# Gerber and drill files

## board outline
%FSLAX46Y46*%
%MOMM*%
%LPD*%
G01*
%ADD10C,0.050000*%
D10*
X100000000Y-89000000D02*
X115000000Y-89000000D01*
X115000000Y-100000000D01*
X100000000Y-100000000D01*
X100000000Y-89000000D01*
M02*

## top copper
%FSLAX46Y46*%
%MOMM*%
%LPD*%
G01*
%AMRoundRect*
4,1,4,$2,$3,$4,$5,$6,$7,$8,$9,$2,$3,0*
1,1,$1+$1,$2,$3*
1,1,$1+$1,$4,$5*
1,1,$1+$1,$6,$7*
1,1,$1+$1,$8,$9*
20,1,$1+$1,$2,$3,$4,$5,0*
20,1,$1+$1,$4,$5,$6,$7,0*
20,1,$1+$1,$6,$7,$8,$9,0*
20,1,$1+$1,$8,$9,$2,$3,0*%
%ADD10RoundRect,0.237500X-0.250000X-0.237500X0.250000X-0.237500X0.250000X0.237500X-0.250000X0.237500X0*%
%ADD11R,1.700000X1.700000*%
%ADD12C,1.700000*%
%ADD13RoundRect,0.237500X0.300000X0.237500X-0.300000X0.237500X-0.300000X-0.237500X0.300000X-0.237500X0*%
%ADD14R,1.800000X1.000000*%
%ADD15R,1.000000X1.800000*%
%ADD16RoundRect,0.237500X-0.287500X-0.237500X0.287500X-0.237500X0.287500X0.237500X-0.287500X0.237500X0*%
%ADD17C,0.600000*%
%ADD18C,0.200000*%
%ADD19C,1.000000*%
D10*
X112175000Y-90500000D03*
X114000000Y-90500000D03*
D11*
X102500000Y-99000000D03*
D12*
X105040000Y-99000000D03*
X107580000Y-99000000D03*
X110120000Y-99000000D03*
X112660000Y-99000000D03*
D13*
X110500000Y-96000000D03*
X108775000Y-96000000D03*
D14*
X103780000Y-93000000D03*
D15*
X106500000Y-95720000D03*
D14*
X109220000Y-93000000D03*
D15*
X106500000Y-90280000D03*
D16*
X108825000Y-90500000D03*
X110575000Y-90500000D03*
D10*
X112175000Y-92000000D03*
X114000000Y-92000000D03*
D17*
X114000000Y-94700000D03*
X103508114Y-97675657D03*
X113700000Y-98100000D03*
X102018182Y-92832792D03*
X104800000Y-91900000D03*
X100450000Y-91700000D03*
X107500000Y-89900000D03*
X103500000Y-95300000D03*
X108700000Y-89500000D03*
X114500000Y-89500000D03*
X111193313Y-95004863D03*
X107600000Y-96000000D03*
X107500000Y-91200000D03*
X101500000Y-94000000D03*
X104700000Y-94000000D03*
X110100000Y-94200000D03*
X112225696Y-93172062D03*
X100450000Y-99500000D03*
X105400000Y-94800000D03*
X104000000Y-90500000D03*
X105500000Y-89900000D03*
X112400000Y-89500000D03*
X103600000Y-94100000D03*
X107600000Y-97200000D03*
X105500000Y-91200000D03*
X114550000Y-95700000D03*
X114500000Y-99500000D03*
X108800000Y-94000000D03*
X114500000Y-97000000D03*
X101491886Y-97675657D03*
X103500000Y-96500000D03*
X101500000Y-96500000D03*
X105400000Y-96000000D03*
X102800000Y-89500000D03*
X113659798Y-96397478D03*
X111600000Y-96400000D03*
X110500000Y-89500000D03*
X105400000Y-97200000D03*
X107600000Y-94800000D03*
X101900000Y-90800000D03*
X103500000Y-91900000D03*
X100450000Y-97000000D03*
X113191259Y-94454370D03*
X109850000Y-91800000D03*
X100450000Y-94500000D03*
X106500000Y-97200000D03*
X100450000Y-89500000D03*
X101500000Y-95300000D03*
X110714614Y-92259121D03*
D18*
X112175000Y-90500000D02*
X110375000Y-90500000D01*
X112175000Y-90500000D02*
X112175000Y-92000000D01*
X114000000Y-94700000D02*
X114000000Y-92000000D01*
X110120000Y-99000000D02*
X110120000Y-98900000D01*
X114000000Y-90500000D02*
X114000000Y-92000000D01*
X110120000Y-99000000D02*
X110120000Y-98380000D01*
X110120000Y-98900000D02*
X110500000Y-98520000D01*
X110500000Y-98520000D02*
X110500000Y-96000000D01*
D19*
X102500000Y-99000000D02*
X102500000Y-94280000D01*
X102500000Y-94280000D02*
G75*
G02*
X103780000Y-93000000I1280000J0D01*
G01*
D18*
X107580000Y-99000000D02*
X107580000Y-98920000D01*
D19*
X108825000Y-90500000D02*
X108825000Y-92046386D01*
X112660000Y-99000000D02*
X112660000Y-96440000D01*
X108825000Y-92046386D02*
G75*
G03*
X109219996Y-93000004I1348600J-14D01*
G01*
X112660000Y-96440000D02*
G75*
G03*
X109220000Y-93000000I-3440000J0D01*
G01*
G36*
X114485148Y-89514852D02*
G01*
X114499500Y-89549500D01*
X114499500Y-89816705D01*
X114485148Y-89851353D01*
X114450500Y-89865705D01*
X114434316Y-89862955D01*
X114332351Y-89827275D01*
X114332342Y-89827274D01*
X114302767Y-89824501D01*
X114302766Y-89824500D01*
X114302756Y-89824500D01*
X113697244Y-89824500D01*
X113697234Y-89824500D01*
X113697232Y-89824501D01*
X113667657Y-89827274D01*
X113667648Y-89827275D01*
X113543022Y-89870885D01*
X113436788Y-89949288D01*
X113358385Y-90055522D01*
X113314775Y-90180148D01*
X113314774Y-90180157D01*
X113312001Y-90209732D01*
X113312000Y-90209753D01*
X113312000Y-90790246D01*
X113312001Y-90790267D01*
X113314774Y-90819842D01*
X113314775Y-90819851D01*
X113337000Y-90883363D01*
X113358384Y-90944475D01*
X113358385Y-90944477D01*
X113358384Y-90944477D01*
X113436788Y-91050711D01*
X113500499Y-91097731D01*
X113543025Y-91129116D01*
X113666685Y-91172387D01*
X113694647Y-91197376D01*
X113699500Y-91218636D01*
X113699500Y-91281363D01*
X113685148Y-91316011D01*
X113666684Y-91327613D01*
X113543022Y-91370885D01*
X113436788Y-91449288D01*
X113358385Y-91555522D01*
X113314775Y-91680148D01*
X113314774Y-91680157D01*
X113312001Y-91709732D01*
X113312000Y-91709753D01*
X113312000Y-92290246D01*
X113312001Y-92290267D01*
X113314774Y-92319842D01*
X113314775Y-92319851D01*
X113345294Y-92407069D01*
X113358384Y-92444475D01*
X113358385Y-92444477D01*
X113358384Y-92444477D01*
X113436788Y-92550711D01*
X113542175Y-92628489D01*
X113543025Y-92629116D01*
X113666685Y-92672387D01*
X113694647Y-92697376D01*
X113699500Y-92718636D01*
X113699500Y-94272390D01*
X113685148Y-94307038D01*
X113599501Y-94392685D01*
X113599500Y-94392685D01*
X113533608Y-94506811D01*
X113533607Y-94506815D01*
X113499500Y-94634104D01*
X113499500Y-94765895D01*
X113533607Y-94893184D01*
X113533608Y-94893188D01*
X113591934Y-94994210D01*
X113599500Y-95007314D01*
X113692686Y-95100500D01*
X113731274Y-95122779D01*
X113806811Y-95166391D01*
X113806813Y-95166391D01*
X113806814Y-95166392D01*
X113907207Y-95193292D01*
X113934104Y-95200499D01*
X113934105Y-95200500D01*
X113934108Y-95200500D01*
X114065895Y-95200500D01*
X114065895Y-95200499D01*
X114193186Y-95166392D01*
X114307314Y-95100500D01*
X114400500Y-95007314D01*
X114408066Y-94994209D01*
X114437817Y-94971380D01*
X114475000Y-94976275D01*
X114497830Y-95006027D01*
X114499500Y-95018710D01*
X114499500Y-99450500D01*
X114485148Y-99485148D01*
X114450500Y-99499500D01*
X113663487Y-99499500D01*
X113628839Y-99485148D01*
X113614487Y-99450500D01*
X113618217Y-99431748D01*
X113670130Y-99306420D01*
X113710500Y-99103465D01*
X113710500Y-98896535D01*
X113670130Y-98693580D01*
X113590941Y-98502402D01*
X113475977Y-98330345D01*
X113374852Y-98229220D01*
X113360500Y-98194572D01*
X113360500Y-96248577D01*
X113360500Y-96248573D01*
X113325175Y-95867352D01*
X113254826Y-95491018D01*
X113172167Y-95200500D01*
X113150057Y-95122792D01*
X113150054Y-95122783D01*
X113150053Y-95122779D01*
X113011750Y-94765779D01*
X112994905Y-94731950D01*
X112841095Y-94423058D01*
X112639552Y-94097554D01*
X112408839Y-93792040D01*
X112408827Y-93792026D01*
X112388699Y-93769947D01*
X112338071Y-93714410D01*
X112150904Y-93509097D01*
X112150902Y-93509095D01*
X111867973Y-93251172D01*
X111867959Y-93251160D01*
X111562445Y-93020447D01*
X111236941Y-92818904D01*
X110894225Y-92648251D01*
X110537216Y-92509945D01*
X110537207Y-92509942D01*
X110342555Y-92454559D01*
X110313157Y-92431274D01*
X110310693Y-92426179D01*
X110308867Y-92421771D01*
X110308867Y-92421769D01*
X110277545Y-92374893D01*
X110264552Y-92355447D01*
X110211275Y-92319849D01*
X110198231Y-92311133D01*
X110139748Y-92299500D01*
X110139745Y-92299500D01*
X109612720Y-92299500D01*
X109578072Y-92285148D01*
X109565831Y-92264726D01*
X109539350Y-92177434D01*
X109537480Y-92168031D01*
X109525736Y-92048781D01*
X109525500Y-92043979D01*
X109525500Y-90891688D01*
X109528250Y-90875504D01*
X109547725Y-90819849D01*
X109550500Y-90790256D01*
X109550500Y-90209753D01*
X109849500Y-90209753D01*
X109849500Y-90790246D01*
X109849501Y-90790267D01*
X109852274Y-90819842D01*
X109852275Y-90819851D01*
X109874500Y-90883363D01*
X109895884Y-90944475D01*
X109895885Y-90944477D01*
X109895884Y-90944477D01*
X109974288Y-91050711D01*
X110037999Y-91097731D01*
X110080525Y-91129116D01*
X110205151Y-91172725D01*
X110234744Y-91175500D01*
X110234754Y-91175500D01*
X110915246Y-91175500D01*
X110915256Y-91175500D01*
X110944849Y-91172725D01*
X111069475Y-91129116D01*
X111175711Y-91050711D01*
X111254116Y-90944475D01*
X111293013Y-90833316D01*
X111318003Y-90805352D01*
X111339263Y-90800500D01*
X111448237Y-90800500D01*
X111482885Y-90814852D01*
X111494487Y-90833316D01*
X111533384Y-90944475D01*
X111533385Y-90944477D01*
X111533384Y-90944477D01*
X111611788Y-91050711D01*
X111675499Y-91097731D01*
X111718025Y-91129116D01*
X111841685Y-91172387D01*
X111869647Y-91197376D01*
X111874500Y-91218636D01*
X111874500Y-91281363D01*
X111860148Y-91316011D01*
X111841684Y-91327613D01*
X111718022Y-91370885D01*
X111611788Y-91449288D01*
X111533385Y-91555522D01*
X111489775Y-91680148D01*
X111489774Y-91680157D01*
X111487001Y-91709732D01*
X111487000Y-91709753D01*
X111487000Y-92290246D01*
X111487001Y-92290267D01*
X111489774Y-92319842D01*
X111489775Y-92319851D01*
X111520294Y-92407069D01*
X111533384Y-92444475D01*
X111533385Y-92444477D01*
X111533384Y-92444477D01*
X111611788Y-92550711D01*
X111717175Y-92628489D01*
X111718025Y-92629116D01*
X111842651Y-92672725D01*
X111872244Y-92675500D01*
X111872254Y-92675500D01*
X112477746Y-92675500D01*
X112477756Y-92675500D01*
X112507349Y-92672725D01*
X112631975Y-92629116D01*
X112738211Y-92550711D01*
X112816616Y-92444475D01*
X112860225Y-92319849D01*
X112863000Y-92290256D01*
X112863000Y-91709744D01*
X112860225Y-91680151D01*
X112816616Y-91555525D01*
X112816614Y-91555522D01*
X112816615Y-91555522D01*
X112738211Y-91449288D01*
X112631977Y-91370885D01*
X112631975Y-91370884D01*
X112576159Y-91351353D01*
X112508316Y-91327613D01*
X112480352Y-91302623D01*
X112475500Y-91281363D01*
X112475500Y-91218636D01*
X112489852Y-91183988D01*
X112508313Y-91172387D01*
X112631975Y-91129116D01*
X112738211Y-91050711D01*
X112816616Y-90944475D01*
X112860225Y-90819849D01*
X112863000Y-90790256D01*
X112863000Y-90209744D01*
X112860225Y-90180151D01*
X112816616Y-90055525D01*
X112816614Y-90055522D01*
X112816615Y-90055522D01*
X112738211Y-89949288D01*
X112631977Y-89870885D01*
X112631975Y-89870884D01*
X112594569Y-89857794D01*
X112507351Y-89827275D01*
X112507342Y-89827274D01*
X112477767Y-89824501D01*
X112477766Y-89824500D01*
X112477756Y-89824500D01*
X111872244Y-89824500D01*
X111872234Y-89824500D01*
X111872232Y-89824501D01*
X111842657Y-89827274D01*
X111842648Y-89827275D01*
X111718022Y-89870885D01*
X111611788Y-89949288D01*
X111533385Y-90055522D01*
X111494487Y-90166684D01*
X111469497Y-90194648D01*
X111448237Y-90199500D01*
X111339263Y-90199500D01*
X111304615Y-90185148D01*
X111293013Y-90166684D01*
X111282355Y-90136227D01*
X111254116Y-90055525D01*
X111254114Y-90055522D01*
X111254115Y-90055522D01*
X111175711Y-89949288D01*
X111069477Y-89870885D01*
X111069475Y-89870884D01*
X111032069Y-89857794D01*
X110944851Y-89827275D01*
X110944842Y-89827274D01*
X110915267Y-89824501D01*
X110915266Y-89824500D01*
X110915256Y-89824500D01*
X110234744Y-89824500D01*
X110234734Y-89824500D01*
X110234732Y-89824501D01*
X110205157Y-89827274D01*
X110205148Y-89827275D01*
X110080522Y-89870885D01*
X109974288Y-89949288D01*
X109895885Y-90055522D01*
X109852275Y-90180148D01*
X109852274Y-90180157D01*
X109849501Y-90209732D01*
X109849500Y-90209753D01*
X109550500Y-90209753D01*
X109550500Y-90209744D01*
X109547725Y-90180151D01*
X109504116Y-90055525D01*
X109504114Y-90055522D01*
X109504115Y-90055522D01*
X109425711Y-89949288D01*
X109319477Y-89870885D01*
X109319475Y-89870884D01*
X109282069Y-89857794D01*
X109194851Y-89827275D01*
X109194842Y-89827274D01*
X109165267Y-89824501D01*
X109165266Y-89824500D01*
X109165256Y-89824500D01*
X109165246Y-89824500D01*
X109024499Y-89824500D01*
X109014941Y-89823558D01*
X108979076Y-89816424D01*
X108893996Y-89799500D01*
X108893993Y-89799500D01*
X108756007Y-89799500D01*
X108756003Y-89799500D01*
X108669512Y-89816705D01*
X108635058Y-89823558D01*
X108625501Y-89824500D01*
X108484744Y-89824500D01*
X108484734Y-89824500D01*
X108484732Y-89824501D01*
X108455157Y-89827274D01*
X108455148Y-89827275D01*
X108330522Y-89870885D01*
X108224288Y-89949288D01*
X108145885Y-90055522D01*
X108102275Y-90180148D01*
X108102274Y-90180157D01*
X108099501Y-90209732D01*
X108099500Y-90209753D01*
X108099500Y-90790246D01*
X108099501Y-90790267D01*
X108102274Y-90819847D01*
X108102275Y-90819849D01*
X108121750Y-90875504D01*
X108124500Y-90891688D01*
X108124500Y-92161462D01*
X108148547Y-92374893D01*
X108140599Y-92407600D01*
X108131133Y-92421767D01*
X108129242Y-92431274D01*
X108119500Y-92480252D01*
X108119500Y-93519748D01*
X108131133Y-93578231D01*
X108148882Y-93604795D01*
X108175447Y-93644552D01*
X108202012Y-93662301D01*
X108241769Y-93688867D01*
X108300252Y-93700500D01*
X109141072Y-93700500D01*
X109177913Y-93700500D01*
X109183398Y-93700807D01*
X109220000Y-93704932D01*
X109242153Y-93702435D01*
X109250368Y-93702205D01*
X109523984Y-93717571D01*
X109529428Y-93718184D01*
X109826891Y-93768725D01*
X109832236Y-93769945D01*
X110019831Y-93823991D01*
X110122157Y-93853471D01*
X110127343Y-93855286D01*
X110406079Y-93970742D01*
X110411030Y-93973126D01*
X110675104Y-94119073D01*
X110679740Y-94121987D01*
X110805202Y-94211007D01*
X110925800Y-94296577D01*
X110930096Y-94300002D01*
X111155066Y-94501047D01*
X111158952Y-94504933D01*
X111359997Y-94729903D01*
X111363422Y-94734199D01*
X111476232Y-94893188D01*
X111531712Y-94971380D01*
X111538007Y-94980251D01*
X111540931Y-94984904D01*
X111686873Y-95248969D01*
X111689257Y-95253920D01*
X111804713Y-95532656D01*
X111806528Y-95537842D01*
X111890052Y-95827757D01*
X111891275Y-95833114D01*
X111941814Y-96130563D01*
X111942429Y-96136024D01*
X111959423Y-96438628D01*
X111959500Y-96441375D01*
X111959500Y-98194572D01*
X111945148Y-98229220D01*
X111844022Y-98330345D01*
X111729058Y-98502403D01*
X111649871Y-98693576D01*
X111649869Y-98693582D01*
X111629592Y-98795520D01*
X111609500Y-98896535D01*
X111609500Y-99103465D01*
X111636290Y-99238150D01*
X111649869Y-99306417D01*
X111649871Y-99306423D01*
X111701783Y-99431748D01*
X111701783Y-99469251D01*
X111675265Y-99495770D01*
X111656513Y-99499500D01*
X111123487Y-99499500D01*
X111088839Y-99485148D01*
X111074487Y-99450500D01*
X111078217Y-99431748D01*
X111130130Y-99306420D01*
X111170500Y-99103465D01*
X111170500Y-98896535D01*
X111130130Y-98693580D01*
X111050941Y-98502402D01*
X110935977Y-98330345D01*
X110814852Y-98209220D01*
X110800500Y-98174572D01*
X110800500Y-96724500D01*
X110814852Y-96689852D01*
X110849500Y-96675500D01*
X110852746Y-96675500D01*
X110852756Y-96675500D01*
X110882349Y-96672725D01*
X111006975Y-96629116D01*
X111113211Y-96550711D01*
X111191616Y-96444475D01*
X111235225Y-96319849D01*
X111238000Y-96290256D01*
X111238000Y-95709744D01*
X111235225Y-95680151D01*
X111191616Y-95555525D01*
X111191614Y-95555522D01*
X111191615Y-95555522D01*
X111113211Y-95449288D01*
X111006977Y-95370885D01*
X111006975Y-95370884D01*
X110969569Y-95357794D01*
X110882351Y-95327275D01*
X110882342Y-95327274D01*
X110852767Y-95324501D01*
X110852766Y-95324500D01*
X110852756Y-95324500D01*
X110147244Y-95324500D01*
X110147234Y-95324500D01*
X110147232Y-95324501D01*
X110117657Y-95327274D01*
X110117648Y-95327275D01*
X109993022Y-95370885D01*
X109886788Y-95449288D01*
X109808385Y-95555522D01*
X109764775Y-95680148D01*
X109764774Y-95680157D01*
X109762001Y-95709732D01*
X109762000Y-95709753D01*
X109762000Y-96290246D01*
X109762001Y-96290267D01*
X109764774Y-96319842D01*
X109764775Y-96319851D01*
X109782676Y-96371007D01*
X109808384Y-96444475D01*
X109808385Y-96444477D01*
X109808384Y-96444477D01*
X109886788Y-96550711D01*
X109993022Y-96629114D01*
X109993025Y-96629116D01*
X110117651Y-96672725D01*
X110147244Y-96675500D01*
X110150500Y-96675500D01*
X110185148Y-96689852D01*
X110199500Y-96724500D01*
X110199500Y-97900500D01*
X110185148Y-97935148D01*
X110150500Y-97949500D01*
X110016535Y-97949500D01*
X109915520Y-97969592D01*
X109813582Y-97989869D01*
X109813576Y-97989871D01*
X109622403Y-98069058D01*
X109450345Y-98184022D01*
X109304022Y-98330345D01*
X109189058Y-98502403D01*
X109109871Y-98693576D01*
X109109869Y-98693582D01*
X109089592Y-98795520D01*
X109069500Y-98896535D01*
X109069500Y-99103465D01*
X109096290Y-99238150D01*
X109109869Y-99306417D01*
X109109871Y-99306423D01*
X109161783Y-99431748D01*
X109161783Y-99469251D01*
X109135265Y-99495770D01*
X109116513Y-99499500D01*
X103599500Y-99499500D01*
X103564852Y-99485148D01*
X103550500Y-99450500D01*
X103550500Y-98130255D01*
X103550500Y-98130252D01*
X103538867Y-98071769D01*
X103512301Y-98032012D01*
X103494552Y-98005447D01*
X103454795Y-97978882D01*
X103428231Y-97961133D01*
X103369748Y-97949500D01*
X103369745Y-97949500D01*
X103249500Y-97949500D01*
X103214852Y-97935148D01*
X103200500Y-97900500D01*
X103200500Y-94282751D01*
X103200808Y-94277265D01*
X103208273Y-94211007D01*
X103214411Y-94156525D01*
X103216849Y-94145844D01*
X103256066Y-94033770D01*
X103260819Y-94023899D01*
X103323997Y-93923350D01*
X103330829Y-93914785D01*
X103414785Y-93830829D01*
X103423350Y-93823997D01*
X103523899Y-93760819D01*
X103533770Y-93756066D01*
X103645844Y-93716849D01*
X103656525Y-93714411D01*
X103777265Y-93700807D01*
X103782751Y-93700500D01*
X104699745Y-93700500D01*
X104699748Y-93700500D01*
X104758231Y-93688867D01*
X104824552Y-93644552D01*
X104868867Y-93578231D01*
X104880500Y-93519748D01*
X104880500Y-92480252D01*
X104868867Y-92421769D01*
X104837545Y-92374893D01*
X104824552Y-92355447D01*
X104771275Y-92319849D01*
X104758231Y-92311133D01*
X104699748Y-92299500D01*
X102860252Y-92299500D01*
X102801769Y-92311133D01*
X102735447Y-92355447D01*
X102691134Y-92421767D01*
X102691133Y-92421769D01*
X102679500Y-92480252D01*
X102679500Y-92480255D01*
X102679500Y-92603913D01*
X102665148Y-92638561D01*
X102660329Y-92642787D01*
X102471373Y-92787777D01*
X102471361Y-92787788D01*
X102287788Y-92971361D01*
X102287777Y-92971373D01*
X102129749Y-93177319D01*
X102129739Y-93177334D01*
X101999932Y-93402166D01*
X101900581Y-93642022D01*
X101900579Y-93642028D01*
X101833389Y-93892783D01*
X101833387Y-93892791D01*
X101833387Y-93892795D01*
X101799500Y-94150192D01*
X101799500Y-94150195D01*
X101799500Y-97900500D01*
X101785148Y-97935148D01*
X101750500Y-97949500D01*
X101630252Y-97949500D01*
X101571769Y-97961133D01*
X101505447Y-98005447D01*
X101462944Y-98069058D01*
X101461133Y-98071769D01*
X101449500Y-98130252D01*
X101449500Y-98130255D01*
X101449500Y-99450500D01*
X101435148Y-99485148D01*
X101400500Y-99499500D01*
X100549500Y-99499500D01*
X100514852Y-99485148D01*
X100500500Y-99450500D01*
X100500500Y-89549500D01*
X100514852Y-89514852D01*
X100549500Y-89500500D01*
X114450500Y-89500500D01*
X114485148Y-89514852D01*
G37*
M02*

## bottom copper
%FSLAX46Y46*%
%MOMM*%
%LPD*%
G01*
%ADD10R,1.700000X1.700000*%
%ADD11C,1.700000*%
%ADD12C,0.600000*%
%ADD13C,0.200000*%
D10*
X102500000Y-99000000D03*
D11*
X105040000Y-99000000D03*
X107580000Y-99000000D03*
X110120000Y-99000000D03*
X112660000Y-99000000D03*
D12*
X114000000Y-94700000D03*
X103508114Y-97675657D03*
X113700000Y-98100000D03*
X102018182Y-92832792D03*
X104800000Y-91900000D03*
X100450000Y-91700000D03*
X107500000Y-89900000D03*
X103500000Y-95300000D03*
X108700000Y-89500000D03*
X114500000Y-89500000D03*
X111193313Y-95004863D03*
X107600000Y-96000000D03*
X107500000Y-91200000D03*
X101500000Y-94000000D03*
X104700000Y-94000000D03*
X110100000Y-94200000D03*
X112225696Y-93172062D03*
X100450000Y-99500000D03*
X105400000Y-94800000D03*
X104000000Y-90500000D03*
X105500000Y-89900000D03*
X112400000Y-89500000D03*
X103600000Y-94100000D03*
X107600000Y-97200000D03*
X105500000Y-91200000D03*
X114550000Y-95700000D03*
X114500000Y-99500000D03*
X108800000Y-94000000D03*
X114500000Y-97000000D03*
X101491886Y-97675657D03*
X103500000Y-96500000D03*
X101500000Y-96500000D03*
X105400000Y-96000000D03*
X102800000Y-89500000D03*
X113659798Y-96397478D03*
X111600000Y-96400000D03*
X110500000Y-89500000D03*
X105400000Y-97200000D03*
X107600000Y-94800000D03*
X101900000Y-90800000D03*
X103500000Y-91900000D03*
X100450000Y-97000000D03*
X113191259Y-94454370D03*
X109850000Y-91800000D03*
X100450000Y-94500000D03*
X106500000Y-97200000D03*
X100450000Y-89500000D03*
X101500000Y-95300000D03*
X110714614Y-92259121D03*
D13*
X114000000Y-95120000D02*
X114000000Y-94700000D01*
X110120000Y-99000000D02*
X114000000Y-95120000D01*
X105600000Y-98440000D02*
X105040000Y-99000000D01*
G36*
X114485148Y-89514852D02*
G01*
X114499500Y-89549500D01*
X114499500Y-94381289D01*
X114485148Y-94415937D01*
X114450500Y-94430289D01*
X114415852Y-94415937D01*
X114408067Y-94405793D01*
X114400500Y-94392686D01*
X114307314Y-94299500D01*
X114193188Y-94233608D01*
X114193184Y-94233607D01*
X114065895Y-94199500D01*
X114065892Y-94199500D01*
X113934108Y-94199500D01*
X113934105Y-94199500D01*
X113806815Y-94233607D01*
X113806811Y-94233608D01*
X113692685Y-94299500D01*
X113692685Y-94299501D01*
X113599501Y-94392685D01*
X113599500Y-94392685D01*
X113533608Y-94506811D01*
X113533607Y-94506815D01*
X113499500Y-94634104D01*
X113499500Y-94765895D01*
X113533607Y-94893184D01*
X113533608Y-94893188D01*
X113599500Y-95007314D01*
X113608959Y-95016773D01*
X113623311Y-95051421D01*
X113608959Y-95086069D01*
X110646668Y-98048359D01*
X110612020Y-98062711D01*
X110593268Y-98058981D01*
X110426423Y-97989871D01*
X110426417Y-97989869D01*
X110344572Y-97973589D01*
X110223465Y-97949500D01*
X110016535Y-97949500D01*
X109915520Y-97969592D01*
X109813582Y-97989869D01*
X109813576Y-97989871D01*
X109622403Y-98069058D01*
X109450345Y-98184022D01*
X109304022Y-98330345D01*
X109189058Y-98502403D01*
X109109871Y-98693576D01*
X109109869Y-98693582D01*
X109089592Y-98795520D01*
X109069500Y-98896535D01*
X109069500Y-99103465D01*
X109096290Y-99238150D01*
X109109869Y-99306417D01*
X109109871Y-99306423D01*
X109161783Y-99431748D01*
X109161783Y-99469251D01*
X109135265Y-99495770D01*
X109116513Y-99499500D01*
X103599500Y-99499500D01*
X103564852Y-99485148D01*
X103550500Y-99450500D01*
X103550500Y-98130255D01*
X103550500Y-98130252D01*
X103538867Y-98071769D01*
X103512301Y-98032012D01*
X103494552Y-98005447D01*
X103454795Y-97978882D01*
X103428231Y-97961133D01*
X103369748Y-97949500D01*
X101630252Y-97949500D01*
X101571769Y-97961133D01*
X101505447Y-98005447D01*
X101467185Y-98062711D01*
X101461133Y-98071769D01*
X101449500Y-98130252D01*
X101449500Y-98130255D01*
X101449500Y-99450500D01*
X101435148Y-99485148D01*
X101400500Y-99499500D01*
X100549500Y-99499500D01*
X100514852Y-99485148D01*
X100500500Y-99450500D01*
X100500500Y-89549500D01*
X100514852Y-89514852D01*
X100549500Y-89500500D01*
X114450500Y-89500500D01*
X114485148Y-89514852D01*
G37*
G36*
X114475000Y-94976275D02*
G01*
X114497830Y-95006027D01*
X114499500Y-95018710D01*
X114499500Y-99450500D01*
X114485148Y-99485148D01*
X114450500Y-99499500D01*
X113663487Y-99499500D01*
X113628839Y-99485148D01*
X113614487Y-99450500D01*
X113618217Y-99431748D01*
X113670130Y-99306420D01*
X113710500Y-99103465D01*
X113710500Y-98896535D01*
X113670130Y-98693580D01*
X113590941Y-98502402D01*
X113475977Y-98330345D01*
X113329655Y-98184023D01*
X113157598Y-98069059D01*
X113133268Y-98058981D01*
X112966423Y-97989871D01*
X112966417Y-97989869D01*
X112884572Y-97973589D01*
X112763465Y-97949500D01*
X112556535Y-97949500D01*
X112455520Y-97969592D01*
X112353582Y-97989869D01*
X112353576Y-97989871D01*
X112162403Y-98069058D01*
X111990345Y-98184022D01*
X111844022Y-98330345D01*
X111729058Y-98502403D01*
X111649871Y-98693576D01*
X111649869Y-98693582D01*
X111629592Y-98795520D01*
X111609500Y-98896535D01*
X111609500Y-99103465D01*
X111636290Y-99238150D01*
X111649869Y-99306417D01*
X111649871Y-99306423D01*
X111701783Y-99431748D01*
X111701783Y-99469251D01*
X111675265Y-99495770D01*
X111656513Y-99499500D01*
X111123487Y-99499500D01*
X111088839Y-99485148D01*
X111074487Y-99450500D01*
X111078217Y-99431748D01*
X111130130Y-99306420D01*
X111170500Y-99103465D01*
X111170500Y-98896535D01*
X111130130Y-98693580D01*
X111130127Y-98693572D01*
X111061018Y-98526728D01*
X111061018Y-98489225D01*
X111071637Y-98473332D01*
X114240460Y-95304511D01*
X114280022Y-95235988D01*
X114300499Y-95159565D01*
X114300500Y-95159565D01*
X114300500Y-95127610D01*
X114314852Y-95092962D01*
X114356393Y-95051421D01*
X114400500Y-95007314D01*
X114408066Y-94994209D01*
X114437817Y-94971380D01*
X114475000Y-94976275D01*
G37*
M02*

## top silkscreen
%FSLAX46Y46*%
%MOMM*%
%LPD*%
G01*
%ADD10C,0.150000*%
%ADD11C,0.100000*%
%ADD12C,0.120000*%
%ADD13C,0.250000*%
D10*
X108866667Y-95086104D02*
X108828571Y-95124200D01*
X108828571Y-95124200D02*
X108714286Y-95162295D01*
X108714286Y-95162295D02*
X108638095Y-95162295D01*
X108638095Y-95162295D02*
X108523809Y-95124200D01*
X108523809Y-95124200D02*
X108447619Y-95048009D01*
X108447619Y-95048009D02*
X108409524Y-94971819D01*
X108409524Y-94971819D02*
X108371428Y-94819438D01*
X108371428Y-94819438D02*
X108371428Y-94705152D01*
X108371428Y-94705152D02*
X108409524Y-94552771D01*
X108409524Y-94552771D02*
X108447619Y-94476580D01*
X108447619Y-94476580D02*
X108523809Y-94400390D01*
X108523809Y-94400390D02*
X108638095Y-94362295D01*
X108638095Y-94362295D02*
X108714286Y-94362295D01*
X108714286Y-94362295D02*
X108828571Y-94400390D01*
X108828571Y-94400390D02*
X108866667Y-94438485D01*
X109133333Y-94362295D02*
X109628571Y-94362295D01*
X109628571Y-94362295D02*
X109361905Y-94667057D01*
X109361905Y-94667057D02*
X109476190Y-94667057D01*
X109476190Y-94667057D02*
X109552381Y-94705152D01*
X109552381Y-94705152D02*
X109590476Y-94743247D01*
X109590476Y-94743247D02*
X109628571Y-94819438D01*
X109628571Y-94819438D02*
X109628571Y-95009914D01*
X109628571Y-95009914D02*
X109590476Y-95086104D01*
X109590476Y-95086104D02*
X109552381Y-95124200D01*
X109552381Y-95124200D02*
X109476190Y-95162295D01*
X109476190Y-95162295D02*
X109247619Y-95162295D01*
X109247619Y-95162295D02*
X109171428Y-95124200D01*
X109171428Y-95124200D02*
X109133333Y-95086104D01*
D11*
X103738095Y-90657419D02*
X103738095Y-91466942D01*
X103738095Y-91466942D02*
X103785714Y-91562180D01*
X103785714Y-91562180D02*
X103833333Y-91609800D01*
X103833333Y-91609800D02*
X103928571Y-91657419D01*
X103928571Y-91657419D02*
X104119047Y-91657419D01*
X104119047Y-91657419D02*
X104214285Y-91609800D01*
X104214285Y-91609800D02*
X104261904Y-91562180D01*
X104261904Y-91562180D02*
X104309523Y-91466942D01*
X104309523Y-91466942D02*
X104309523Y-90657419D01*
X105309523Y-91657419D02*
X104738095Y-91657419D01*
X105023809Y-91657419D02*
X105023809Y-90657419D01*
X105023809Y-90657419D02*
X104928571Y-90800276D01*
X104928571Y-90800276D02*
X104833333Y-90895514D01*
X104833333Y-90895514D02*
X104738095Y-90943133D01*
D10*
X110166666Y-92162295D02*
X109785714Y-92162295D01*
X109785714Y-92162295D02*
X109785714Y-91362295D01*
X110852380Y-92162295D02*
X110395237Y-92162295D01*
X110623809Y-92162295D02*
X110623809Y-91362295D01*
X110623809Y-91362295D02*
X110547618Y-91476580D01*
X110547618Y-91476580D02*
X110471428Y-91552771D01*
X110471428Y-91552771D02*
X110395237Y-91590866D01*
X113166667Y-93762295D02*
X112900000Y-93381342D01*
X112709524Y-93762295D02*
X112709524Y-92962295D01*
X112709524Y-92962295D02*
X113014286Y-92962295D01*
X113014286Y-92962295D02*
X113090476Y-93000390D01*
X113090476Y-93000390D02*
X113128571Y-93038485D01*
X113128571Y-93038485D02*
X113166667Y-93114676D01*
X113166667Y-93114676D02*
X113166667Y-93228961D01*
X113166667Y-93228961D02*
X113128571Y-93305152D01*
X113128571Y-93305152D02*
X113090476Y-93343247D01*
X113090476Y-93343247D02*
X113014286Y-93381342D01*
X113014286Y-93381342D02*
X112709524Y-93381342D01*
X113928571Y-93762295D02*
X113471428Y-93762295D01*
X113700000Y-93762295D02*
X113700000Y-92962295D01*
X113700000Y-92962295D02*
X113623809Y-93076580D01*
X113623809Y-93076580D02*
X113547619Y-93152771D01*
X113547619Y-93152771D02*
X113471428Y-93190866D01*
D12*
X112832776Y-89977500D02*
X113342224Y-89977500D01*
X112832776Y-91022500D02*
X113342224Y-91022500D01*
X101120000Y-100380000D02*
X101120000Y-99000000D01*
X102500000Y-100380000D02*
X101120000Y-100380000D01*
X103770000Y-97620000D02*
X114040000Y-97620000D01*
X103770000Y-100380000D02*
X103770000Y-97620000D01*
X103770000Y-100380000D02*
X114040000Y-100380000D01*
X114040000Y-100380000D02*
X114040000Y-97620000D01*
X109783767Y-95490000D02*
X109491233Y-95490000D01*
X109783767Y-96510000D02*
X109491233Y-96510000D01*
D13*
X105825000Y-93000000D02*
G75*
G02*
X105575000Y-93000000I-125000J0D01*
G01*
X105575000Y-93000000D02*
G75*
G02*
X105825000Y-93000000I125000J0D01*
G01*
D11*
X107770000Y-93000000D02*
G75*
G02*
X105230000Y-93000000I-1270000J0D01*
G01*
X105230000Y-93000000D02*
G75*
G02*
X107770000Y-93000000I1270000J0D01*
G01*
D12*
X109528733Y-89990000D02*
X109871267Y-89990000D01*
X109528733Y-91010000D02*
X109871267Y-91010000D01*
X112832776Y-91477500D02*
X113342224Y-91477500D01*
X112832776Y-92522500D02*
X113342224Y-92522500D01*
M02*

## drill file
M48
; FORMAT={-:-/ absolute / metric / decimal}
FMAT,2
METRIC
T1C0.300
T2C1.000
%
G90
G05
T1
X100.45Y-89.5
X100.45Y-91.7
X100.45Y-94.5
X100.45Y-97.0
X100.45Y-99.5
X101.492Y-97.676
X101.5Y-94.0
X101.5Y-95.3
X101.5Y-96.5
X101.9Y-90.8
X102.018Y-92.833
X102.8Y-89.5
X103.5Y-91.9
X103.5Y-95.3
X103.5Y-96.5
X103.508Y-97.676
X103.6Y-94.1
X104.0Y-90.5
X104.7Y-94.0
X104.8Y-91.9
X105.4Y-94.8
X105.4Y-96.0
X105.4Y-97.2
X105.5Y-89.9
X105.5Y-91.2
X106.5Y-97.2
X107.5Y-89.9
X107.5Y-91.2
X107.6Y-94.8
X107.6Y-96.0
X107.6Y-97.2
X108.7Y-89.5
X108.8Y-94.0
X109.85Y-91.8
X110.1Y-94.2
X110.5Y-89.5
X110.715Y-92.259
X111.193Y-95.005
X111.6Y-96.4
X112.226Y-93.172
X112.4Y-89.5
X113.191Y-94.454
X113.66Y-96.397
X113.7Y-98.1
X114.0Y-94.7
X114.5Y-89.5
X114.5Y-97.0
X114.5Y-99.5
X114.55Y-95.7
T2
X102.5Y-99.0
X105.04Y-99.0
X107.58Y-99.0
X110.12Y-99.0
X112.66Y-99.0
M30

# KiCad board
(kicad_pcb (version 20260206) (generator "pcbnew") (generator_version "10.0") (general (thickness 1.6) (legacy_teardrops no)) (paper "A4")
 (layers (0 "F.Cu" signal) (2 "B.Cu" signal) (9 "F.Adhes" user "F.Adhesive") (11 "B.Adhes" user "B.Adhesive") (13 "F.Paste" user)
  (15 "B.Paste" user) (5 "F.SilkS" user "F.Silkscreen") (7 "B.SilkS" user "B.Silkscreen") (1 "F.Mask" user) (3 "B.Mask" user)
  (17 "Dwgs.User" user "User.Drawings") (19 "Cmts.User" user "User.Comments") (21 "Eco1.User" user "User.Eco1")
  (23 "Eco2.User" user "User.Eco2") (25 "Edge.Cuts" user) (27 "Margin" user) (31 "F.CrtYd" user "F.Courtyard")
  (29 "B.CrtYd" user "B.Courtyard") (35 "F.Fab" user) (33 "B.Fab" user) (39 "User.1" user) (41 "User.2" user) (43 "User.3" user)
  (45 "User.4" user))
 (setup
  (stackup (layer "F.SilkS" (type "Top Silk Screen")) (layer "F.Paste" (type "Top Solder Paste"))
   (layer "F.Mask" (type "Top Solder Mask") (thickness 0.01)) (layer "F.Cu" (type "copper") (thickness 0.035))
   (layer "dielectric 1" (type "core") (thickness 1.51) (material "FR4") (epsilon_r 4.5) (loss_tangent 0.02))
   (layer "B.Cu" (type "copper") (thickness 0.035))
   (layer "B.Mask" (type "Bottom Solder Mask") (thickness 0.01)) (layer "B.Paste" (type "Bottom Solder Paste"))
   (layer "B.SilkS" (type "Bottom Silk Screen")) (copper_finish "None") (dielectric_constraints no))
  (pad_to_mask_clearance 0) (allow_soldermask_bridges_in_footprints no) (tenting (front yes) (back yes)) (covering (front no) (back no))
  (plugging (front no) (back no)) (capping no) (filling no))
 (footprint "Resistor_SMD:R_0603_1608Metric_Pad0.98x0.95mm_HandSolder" (layer "F.Cu") (at 113.0875 90.5)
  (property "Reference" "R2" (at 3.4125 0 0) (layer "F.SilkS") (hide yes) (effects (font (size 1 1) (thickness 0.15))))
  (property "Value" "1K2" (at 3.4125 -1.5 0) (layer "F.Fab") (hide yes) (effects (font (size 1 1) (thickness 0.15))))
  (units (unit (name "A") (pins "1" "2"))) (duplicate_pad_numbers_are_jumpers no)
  (fp_line (start -0.254724 -0.5225) (end 0.254724 -0.5225) (stroke (width 0.12) (type solid)) (layer "F.SilkS"))
  (fp_line (start -0.254724 0.5225) (end 0.254724 0.5225) (stroke (width 0.12) (type solid)) (layer "F.SilkS"))
  (pad "1" smd roundrect (at -0.9125 0) (size 0.975 0.95) (layers "F.Cu" "F.Mask" "F.Paste") (roundrect_rratio 0.25) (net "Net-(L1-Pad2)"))
  (pad "2" smd roundrect (at 0.9125 0) (size 0.975 0.95) (layers "F.Cu" "F.Mask" "F.Paste") (roundrect_rratio 0.25) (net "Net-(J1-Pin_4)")))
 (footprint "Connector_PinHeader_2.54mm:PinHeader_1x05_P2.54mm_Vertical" (layer "F.Cu") (at 102.5 99 90)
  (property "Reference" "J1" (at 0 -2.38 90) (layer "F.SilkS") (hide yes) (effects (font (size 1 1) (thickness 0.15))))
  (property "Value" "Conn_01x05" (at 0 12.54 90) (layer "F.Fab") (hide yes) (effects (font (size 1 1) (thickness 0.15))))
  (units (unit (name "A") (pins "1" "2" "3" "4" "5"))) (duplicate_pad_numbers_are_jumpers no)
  (fp_line (start -1.38 -1.38) (end 0 -1.38) (stroke (width 0.12) (type solid)) (layer "F.SilkS"))
  (fp_line (start -1.38 0) (end -1.38 -1.38) (stroke (width 0.12) (type solid)) (layer "F.SilkS"))
  (fp_line (start 1.38 1.27) (end 1.38 11.54) (stroke (width 0.12) (type solid)) (layer "F.SilkS"))
  (fp_line (start -1.38 1.27) (end 1.38 1.27) (stroke (width 0.12) (type solid)) (layer "F.SilkS"))
  (fp_line (start -1.38 1.27) (end -1.38 11.54) (stroke (width 0.12) (type solid)) (layer "F.SilkS"))
  (fp_line (start -1.38 11.54) (end 1.38 11.54) (stroke (width 0.12) (type solid)) (layer "F.SilkS"))
  (pad "1" thru_hole rect (at 0 0 90) (size 1.7 1.7) (drill 1) (layers "*.Cu" "*.Mask") (remove_unused_layers no) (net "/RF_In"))
  (pad "2" thru_hole circle (at 0 2.54 90) (size 1.7 1.7) (drill 1) (layers "*.Cu" "*.Mask") (remove_unused_layers no) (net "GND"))
  (pad "3" thru_hole circle (at 0 5.08 90) (size 1.7 1.7) (drill 1) (layers "*.Cu" "*.Mask") (remove_unused_layers no) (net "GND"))
  (pad "4" thru_hole circle (at 0 7.62 90) (size 1.7 1.7) (drill 1) (layers "*.Cu" "*.Mask") (remove_unused_layers no)
   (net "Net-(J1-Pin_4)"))
  (pad "5" thru_hole circle (at 0 10.16 90) (size 1.7 1.7) (drill 1) (layers "*.Cu" "*.Mask") (remove_unused_layers no) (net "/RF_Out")))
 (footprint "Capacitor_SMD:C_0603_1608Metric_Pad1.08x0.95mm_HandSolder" (layer "F.Cu") (at 109.6375 96 180)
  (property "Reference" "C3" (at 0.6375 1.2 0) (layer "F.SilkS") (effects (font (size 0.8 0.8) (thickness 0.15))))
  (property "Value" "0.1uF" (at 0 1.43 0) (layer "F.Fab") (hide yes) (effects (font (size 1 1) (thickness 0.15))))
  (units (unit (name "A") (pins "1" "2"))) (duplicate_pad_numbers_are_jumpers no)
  (fp_line (start -0.146267 0.51) (end 0.146267 0.51) (stroke (width 0.12) (type solid)) (layer "F.SilkS"))
  (fp_line (start -0.146267 -0.51) (end 0.146267 -0.51) (stroke (width 0.12) (type solid)) (layer "F.SilkS"))
  (pad "1" smd roundrect (at -0.8625 0 180) (size 1.075 0.95) (layers "F.Cu" "F.Mask" "F.Paste") (roundrect_rratio 0.25)
   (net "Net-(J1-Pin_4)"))
  (pad "2" smd roundrect (at 0.8625 0 180) (size 1.075 0.95) (layers "F.Cu" "F.Mask" "F.Paste") (roundrect_rratio 0.25) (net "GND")))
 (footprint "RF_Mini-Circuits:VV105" (layer "F.Cu") (at 106.5 93 -90)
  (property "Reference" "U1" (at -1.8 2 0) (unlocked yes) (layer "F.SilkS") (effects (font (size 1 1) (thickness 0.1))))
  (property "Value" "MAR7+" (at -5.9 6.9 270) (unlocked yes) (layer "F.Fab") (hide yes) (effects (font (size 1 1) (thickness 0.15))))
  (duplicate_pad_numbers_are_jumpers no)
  (fp_circle (center 0 0.8) (end 0.2 0.8) (stroke (width 0.1) (type default)) (fill yes) (layer "F.SilkS"))
  (fp_circle (center 0 0) (end 1.27 0) (stroke (width 0.1) (type solid)) (fill no) (layer "F.SilkS"))
  (pad "1" smd rect (at 0 2.72 180) (size 1.8 1) (layers "F.Cu" "F.Mask") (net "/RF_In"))
  (pad "2" smd rect (at 2.72 0 270) (size 1.8 1) (layers "F.Cu" "F.Mask") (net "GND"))
  (pad "3" smd rect (at 0 -2.72 180) (size 1.8 1) (layers "F.Cu" "F.Mask") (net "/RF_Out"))
  (pad "4" smd rect (at -2.72 0 270) (size 1.8 1) (layers "F.Cu" "F.Mask") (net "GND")))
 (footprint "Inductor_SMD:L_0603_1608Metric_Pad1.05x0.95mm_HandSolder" (layer "F.Cu") (at 109.7 90.5)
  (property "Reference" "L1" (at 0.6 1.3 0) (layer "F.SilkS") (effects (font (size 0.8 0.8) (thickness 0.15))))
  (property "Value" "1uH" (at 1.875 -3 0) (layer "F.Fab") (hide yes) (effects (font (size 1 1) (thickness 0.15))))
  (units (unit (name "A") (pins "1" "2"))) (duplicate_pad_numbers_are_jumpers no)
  (fp_line (start -0.171267 -0.51) (end 0.171267 -0.51) (stroke (width 0.12) (type solid)) (layer "F.SilkS"))
  (fp_line (start -0.171267 0.51) (end 0.171267 0.51) (stroke (width 0.12) (type solid)) (layer "F.SilkS"))
  (pad "1" smd roundrect (at -0.875 0) (size 1.05 0.95) (layers "F.Cu" "F.Mask" "F.Paste") (roundrect_rratio 0.25) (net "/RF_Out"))
  (pad "2" smd roundrect (at 0.875 0) (size 1.05 0.95) (layers "F.Cu" "F.Mask" "F.Paste") (roundrect_rratio 0.25) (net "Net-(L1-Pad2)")))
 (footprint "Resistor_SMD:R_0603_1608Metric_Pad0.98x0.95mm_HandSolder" (layer "F.Cu") (at 113.0875 92)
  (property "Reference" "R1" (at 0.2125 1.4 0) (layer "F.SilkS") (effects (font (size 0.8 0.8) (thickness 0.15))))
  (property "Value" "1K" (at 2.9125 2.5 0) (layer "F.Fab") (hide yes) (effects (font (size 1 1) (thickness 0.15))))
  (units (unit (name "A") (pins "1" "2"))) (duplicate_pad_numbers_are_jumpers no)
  (fp_line (start -0.254724 -0.5225) (end 0.254724 -0.5225) (stroke (width 0.12) (type solid)) (layer "F.SilkS"))
  (fp_line (start -0.254724 0.5225) (end 0.254724 0.5225) (stroke (width 0.12) (type solid)) (layer "F.SilkS"))
  (pad "1" smd roundrect (at -0.9125 0) (size 0.975 0.95) (layers "F.Cu" "F.Mask" "F.Paste") (roundrect_rratio 0.25) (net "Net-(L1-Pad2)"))
  (pad "2" smd roundrect (at 0.9125 0) (size 0.975 0.95) (layers "F.Cu" "F.Mask" "F.Paste") (roundrect_rratio 0.25) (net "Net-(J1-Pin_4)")))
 (gr_rect (start 100 89) (end 115 100) (stroke (width 0.05) (type default)) (fill no) (layer "Edge.Cuts"))
 (segment (start 112.175 90.5) (end 110.375 90.5) (width 0.2) (layer "F.Cu") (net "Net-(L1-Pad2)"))
 (segment (start 112.175 90.5) (end 112.175 92) (width 0.2) (layer "F.Cu") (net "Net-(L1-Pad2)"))
 (segment (start 114 94.7) (end 114 92) (width 0.2) (layer "F.Cu") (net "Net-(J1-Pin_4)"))
 (segment (start 110.12 99) (end 110.12 98.9) (width 0.2) (layer "F.Cu") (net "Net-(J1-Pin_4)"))
 (segment (start 114 90.5) (end 114 92) (width 0.2) (layer "F.Cu") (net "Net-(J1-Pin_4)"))
 (segment (start 110.12 99) (end 110.12 98.38) (width 0.2) (layer "F.Cu") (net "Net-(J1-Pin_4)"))
 (segment (start 110.12 98.9) (end 110.5 98.52) (width 0.2) (layer "F.Cu") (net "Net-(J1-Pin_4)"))
 (segment (start 110.5 98.52) (end 110.5 96) (width 0.2) (layer "F.Cu") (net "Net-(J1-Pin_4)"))
 (via (at 114 94.7) (size 0.6) (drill 0.3) (layers "F.Cu" "B.Cu") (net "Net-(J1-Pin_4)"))
 (segment (start 114 95.12) (end 114 94.7) (width 0.2) (layer "B.Cu") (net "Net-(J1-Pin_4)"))
 (segment (start 110.12 99) (end 114 95.12) (width 0.2) (layer "B.Cu") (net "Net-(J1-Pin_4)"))
 (segment (start 102.5 99) (end 102.5 94.28) (width 1) (layer "F.Cu") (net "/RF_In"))
 (arc (start 102.5 94.28) (mid 102.874903 93.374903) (end 103.78 93) (width 1) (layer "F.Cu") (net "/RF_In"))
 (segment (start 107.58 99) (end 107.58 98.92) (width 0.2) (layer "F.Cu") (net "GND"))
 (via (at 103.508114 97.675657) (size 0.6) (drill 0.3) (layers "F.Cu" "B.Cu") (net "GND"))
 (via (at 113.7 98.1) (size 0.6) (drill 0.3) (layers "F.Cu" "B.Cu") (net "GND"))
 (via (at 102.018182 92.832792) (size 0.6) (drill 0.3) (layers "F.Cu" "B.Cu") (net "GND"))
 (via (at 104.8 91.9) (size 0.6) (drill 0.3) (layers "F.Cu" "B.Cu") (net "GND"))
 (via (at 100.45 91.7) (size 0.6) (drill 0.3) (layers "F.Cu" "B.Cu") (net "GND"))
 (via (at 107.5 89.9) (size 0.6) (drill 0.3) (layers "F.Cu" "B.Cu") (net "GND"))
 (via (at 103.5 95.3) (size 0.6) (drill 0.3) (layers "F.Cu" "B.Cu") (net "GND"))
 (via (at 108.7 89.5) (size 0.6) (drill 0.3) (layers "F.Cu" "B.Cu") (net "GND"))
 (via (at 114.5 89.5) (size 0.6) (drill 0.3) (layers "F.Cu" "B.Cu") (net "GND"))
 (via (at 111.193313 95.004863) (size 0.6) (drill 0.3) (layers "F.Cu" "B.Cu") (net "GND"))
 (via (at 107.6 96) (size 0.6) (drill 0.3) (layers "F.Cu" "B.Cu") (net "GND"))
 (via (at 107.5 91.2) (size 0.6) (drill 0.3) (layers "F.Cu" "B.Cu") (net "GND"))
 (via (at 101.5 94) (size 0.6) (drill 0.3) (layers "F.Cu" "B.Cu") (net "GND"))
 (via (at 104.7 94) (size 0.6) (drill 0.3) (layers "F.Cu" "B.Cu") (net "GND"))
 (via (at 110.1 94.2) (size 0.6) (drill 0.3) (layers "F.Cu" "B.Cu") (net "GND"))
 (via (at 112.225696 93.172062) (size 0.6) (drill 0.3) (layers "F.Cu" "B.Cu") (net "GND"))
 (via (at 100.45 99.5) (size 0.6) (drill 0.3) (layers "F.Cu" "B.Cu") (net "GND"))
 (via (at 105.4 94.8) (size 0.6) (drill 0.3) (layers "F.Cu" "B.Cu") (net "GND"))
 (via (at 104 90.5) (size 0.6) (drill 0.3) (layers "F.Cu" "B.Cu") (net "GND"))
 (via (at 105.5 89.9) (size 0.6) (drill 0.3) (layers "F.Cu" "B.Cu") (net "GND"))
 (via (at 112.4 89.5) (size 0.6) (drill 0.3) (layers "F.Cu" "B.Cu") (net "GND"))
 (via (at 103.6 94.1) (size 0.6) (drill 0.3) (layers "F.Cu" "B.Cu") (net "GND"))
 (via (at 107.6 97.2) (size 0.6) (drill 0.3) (layers "F.Cu" "B.Cu") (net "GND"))
 (via (at 105.5 91.2) (size 0.6) (drill 0.3) (layers "F.Cu" "B.Cu") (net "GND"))
 (via (at 114.55 95.7) (size 0.6) (drill 0.3) (layers "F.Cu" "B.Cu") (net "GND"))
 (via (at 114.5 99.5) (size 0.6) (drill 0.3) (layers "F.Cu" "B.Cu") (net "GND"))
 (via (at 108.8 94) (size 0.6) (drill 0.3) (layers "F.Cu" "B.Cu") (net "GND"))
 (via (at 114.5 97) (size 0.6) (drill 0.3) (layers "F.Cu" "B.Cu") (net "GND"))
 (via (at 101.491886 97.675657) (size 0.6) (drill 0.3) (layers "F.Cu" "B.Cu") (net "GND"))
 (via (at 103.5 96.5) (size 0.6) (drill 0.3) (layers "F.Cu" "B.Cu") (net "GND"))
 (via (at 101.5 96.5) (size 0.6) (drill 0.3) (layers "F.Cu" "B.Cu") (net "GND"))
 (via (at 105.4 96) (size 0.6) (drill 0.3) (layers "F.Cu" "B.Cu") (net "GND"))
 (via (at 102.8 89.5) (size 0.6) (drill 0.3) (layers "F.Cu" "B.Cu") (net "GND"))
 (via (at 113.659798 96.397478) (size 0.6) (drill 0.3) (layers "F.Cu" "B.Cu") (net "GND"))
 (via (at 111.6 96.4) (size 0.6) (drill 0.3) (layers "F.Cu" "B.Cu") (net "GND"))
 (via (at 110.5 89.5) (size 0.6) (drill 0.3) (layers "F.Cu" "B.Cu") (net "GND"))
 (via (at 105.4 97.2) (size 0.6) (drill 0.3) (layers "F.Cu" "B.Cu") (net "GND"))
 (via (at 107.6 94.8) (size 0.6) (drill 0.3) (layers "F.Cu" "B.Cu") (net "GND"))
 (via (at 101.9 90.8) (size 0.6) (drill 0.3) (layers "F.Cu" "B.Cu") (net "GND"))
 (via (at 103.5 91.9) (size 0.6) (drill 0.3) (layers "F.Cu" "B.Cu") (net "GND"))
 (via (at 100.45 97) (size 0.6) (drill 0.3) (layers "F.Cu" "B.Cu") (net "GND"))
 (via (at 113.191259 94.45437) (size 0.6) (drill 0.3) (layers "F.Cu" "B.Cu") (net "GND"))
 (via (at 109.85 91.8) (size 0.6) (drill 0.3) (layers "F.Cu" "B.Cu") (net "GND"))
 (via (at 100.45 94.5) (size 0.6) (drill 0.3) (layers "F.Cu" "B.Cu") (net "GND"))
 (via (at 106.5 97.2) (size 0.6) (drill 0.3) (layers "F.Cu" "B.Cu") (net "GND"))
 (via (at 100.45 89.5) (size 0.6) (drill 0.3) (layers "F.Cu" "B.Cu") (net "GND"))
 (via (at 101.5 95.3) (size 0.6) (drill 0.3) (layers "F.Cu" "B.Cu") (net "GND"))
 (via (at 110.714614 92.259121) (size 0.6) (drill 0.3) (layers "F.Cu" "B.Cu") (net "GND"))
 (segment (start 105.6 98.44) (end 105.04 99) (width 0.2) (layer "B.Cu") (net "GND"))
 (segment (start 108.825 90.5) (end 108.825 92.046386) (width 1) (layer "F.Cu") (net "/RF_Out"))
 (segment (start 112.66 99) (end 112.66 96.44) (width 1) (layer "F.Cu") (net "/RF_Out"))
 (arc (start 108.825 92.046386) (mid 108.927657 92.562478) (end 109.22 93) (width 1) (layer "F.Cu") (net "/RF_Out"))
 (arc (start 112.66 96.44) (mid 111.652447 94.007553) (end 109.22 93) (width 1) (layer "F.Cu") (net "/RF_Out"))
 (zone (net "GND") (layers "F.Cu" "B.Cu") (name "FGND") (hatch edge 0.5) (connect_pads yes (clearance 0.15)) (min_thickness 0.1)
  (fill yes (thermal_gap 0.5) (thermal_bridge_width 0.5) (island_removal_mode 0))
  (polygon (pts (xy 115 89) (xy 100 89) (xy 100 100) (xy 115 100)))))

